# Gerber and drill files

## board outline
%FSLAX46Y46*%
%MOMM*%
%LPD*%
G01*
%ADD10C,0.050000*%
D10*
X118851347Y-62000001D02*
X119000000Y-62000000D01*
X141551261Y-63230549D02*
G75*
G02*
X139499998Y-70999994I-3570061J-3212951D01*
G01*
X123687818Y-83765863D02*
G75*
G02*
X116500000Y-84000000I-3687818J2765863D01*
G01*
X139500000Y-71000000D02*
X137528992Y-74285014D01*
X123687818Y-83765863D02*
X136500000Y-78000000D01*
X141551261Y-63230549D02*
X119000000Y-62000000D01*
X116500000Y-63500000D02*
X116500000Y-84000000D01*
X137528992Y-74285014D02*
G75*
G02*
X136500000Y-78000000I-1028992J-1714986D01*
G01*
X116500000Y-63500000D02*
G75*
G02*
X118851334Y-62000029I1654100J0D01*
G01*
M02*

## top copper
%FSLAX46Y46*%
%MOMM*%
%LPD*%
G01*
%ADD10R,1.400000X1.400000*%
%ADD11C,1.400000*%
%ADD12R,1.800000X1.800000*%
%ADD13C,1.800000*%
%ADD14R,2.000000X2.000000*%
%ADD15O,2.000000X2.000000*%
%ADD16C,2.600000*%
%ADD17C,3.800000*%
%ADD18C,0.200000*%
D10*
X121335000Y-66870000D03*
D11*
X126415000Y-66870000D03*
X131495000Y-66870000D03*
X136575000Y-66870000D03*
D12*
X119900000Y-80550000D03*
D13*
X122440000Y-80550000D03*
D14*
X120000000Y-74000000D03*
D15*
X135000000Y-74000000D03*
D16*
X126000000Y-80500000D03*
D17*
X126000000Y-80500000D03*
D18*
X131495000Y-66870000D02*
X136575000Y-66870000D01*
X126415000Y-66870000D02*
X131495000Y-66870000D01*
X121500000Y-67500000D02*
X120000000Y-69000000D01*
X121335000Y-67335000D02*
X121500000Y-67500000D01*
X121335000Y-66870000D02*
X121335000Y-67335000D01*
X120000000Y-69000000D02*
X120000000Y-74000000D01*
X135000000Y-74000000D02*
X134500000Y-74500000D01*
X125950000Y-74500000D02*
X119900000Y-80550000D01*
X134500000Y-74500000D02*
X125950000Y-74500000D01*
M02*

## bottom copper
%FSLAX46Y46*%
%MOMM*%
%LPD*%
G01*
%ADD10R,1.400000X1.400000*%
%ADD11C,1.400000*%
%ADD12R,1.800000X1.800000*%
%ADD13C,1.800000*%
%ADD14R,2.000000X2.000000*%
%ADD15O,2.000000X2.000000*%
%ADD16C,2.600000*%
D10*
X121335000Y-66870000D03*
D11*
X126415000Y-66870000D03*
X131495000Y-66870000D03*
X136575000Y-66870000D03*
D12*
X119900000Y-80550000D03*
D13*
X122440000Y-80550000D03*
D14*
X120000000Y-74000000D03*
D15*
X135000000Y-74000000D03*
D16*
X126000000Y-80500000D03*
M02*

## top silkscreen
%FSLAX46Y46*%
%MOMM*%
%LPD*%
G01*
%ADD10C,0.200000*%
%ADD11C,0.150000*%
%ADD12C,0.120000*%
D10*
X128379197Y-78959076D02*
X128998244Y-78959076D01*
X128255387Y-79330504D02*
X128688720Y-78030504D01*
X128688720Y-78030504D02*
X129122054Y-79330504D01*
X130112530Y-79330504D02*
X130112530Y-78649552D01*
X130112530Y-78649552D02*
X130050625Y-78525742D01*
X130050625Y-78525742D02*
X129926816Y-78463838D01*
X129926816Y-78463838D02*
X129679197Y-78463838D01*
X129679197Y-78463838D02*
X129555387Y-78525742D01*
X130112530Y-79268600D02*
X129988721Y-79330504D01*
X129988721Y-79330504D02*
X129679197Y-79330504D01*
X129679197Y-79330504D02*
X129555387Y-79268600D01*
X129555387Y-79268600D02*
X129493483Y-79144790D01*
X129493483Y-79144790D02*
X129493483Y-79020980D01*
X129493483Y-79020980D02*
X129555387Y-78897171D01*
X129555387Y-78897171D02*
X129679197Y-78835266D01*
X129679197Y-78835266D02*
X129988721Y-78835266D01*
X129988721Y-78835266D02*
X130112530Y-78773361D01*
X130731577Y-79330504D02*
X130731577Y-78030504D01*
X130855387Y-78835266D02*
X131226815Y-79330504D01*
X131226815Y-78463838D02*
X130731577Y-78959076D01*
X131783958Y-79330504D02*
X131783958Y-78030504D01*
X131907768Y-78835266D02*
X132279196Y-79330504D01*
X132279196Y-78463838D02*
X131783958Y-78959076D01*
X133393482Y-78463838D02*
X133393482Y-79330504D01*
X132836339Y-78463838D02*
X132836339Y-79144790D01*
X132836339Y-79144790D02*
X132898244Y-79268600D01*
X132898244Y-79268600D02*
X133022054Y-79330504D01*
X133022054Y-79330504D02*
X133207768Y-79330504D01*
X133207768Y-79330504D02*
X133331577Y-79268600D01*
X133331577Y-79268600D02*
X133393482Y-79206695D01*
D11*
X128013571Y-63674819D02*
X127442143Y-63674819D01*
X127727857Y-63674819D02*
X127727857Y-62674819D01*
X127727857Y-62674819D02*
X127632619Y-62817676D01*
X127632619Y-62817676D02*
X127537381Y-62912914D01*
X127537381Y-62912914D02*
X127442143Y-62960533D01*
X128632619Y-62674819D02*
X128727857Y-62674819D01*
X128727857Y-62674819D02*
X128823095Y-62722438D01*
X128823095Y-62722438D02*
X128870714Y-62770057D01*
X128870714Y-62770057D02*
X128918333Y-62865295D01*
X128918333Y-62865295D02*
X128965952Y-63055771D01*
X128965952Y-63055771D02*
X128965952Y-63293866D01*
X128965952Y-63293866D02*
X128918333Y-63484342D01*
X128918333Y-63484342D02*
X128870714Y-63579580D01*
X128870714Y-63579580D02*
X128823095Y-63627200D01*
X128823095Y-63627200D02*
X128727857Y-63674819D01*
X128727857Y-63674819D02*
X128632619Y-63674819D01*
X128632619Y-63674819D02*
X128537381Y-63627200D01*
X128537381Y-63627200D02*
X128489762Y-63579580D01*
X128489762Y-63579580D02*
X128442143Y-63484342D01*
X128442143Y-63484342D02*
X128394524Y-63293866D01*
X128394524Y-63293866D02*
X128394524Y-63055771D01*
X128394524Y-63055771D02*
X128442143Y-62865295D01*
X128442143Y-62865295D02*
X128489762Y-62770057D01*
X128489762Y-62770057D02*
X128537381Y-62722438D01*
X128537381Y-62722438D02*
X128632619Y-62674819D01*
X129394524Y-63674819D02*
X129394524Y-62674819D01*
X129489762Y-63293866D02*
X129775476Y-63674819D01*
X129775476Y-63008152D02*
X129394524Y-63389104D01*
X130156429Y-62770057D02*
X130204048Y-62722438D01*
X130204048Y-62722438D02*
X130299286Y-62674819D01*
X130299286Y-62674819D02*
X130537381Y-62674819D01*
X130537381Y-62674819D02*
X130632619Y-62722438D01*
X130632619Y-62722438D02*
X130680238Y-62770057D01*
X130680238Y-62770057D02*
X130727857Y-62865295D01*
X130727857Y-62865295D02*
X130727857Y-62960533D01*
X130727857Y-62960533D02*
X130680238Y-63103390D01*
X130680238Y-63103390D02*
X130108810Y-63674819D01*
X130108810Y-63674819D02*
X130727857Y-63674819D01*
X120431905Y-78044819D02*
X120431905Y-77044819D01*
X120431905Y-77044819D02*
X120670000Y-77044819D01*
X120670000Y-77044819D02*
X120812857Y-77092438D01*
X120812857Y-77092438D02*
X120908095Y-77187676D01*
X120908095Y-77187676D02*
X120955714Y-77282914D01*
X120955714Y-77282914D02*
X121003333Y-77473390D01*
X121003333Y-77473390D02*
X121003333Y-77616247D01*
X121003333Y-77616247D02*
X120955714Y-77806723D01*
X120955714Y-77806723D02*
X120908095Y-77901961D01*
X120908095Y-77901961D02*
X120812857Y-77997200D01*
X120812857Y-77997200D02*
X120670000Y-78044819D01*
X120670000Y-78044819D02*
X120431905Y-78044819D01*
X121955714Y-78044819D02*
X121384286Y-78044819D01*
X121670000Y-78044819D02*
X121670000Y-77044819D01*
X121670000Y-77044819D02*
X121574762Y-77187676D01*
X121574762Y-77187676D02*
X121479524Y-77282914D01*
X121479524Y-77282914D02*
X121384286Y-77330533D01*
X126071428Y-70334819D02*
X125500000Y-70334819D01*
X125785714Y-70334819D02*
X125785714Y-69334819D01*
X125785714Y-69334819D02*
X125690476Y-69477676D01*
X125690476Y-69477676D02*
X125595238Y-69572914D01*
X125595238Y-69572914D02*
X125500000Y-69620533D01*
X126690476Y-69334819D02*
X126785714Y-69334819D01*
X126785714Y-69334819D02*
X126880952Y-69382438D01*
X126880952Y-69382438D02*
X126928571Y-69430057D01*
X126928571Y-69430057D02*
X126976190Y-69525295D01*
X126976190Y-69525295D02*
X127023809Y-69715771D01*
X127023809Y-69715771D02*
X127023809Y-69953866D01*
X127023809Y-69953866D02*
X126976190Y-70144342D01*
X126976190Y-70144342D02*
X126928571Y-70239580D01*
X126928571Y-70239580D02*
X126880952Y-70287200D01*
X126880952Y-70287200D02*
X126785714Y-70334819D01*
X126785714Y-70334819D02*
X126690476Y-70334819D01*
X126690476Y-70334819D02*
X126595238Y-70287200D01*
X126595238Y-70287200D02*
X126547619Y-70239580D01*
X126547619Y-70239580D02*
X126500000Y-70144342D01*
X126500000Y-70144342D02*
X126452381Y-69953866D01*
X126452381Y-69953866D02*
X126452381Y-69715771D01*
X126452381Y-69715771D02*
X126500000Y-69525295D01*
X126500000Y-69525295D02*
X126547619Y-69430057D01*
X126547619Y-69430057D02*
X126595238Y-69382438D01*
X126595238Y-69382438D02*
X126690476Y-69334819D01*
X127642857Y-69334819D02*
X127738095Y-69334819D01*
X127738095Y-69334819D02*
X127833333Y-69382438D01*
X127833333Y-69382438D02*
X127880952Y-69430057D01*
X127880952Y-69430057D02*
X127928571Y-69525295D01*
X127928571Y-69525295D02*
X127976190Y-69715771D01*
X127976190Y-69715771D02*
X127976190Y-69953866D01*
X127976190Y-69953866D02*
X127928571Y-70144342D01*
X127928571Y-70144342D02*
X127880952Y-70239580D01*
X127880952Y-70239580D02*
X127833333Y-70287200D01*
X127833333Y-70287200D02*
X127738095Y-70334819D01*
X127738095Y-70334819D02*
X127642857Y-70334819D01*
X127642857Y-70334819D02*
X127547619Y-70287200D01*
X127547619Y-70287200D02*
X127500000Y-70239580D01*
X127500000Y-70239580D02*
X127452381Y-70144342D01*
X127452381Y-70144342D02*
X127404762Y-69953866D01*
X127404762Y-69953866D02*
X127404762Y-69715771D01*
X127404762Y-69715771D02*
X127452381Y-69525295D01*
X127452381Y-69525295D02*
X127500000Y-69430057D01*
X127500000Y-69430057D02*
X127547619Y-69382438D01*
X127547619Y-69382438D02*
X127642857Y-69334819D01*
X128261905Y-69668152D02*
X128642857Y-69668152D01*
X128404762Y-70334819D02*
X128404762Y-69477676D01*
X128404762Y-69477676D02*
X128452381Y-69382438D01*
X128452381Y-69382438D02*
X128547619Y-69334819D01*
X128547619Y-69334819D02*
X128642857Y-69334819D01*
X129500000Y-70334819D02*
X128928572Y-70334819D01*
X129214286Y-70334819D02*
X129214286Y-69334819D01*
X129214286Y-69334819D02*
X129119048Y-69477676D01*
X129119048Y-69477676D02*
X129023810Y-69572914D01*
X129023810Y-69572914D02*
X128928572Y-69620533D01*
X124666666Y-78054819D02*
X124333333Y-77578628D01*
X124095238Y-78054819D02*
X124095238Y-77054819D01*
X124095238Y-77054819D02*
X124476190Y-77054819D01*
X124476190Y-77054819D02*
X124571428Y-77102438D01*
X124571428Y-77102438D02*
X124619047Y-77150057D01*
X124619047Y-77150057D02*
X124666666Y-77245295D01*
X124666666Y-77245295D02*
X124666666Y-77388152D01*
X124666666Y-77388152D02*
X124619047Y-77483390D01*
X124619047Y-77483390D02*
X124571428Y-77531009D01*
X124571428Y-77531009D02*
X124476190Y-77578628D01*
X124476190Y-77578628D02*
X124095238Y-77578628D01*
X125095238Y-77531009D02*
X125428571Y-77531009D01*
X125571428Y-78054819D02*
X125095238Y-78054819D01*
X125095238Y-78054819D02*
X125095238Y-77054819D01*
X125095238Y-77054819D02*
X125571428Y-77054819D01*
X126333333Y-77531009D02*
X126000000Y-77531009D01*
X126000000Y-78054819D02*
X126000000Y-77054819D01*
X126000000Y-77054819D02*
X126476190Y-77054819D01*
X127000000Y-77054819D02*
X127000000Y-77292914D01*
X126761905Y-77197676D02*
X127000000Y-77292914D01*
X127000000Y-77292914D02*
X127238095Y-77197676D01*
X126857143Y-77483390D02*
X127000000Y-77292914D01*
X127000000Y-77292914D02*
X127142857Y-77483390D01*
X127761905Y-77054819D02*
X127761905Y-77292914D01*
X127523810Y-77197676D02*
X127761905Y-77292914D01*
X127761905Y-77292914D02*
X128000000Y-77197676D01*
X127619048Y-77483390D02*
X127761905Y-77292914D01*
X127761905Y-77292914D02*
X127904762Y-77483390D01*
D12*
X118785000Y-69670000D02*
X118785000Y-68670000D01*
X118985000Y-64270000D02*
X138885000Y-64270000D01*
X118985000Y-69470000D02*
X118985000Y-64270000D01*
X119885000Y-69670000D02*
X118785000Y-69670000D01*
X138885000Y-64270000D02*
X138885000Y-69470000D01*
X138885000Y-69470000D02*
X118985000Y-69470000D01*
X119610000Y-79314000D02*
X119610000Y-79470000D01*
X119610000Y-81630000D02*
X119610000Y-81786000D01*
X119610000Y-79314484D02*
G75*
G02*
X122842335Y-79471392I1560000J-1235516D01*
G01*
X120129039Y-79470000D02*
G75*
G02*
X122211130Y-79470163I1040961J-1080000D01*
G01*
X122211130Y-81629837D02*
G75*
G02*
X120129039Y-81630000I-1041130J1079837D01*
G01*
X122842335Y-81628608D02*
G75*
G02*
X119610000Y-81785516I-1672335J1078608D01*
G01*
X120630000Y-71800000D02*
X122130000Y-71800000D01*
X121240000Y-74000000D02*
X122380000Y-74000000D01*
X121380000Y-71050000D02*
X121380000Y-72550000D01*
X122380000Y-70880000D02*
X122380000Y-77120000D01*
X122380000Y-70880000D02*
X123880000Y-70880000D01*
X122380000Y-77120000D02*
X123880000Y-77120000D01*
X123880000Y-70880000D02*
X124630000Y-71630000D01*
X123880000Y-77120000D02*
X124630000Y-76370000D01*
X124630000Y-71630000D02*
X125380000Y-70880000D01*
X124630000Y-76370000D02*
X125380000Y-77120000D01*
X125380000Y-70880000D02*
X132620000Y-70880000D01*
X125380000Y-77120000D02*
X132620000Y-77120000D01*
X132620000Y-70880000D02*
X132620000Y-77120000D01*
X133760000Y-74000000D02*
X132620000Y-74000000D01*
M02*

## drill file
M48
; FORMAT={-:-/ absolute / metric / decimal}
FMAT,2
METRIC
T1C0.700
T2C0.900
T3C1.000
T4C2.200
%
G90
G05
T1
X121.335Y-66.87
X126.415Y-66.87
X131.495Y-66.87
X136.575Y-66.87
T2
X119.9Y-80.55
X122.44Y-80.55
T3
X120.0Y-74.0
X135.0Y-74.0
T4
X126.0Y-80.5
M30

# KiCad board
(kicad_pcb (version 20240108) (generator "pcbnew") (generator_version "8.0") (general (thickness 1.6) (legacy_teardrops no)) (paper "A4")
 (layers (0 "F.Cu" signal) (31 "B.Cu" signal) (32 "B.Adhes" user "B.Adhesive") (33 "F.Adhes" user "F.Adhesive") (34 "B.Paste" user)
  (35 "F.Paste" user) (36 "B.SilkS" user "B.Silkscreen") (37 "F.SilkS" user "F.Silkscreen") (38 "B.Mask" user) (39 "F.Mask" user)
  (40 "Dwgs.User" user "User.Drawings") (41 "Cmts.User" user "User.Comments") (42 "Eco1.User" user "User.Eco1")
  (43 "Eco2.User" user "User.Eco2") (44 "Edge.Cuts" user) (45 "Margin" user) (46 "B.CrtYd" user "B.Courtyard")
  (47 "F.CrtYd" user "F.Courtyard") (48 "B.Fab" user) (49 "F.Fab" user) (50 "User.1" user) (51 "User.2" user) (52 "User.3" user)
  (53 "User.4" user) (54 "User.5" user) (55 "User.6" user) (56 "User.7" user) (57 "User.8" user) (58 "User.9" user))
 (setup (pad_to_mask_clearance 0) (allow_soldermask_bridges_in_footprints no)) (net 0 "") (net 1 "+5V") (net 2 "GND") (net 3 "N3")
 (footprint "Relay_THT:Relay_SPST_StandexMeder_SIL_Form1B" (layer "F.Cu") (at 121.335 66.87)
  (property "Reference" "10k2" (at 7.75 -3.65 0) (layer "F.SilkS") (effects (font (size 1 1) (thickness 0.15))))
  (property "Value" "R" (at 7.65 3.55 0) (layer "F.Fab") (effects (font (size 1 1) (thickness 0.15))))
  (fp_line (start -2.55 2.8) (end -2.55 1.8) (stroke (width 0.12) (type solid)) (layer "F.SilkS"))
  (fp_line (start -2.35 -2.6) (end 17.55 -2.6) (stroke (width 0.12) (type solid)) (layer "F.SilkS"))
  (fp_line (start -2.35 2.6) (end -2.35 -2.6) (stroke (width 0.12) (type solid)) (layer "F.SilkS"))
  (fp_line (start -1.45 2.8) (end -2.55 2.8) (stroke (width 0.12) (type solid)) (layer "F.SilkS"))
  (fp_line (start 17.55 -2.6) (end 17.55 2.6) (stroke (width 0.12) (type solid)) (layer "F.SilkS"))
  (fp_line (start 17.55 2.6) (end -2.35 2.6) (stroke (width 0.12) (type solid)) (layer "F.SilkS"))
  (pad "1" thru_hole rect (at 0 0) (size 1.4 1.4) (drill 0.7) (layers "*.Cu" "*.Mask") (remove_unused_layers no) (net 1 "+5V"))
  (pad "3" thru_hole circle (at 5.08 0) (size 1.4 1.4) (drill 0.7) (layers "*.Cu" "*.Mask") (remove_unused_layers no))
  (pad "5" thru_hole circle (at 10.16 0) (size 1.4 1.4) (drill 0.7) (layers "*.Cu" "*.Mask") (remove_unused_layers no))
  (pad "7" thru_hole circle (at 15.24 0) (size 1.4 1.4) (drill 0.7) (layers "*.Cu" "*.Mask") (remove_unused_layers no)))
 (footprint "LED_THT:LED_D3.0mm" (layer "F.Cu") (at 119.9 80.55)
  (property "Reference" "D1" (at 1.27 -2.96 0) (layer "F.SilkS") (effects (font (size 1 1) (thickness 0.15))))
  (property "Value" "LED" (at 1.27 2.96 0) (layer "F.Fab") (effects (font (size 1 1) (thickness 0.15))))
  (fp_line (start -0.29 -1.236) (end -0.29 -1.08) (stroke (width 0.12) (type solid)) (layer "F.SilkS"))
  (fp_line (start -0.29 1.08) (end -0.29 1.236) (stroke (width 0.12) (type solid)) (layer "F.SilkS"))
  (fp_arc (start -0.29 -1.235516) (mid 1.366487 -1.987659) (end 2.942335 -1.078608) (stroke (width 0.12) (type solid)) (layer "F.SilkS"))
  (fp_arc (start 0.229039 -1.08) (mid 1.270117 -1.5) (end 2.31113 -1.079837) (stroke (width 0.12) (type solid)) (layer "F.SilkS"))
  (fp_arc (start 2.31113 1.079837) (mid 1.270117 1.5) (end 0.229039 1.08) (stroke (width 0.12) (type solid)) (layer "F.SilkS"))
  (fp_arc (start 2.942335 1.078608) (mid 1.366487 1.987659) (end -0.29 1.235516) (stroke (width 0.12) (type solid)) (layer "F.SilkS"))
  (pad "1" thru_hole rect (at 0 0) (size 1.8 1.8) (drill 0.9) (layers "*.Cu" "*.Mask") (remove_unused_layers no) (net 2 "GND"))
  (pad "2" thru_hole circle (at 2.54 0) (size 1.8 1.8) (drill 0.9) (layers "*.Cu" "*.Mask") (remove_unused_layers no) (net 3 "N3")))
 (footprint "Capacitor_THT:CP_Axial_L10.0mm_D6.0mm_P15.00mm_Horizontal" (layer "F.Cu") (at 120 74)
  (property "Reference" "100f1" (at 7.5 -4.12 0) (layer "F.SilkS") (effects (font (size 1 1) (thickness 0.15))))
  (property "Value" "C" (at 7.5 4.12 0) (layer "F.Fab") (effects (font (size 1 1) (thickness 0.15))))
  (fp_line (start 0.63 -2.2) (end 2.13 -2.2) (stroke (width 0.12) (type solid)) (layer "F.SilkS"))
  (fp_line (start 1.24 0) (end 2.38 0) (stroke (width 0.12) (type solid)) (layer "F.SilkS"))
  (fp_line (start 1.38 -2.95) (end 1.38 -1.45) (stroke (width 0.12) (type solid)) (layer "F.SilkS"))
  (fp_line (start 2.38 -3.12) (end 2.38 3.12) (stroke (width 0.12) (type solid)) (layer "F.SilkS"))
  (fp_line (start 2.38 -3.12) (end 3.88 -3.12) (stroke (width 0.12) (type solid)) (layer "F.SilkS"))
  (fp_line (start 2.38 3.12) (end 3.88 3.12) (stroke (width 0.12) (type solid)) (layer "F.SilkS"))
  (fp_line (start 3.88 -3.12) (end 4.63 -2.37) (stroke (width 0.12) (type solid)) (layer "F.SilkS"))
  (fp_line (start 3.88 3.12) (end 4.63 2.37) (stroke (width 0.12) (type solid)) (layer "F.SilkS"))
  (fp_line (start 4.63 -2.37) (end 5.38 -3.12) (stroke (width 0.12) (type solid)) (layer "F.SilkS"))
  (fp_line (start 4.63 2.37) (end 5.38 3.12) (stroke (width 0.12) (type solid)) (layer "F.SilkS"))
  (fp_line (start 5.38 -3.12) (end 12.62 -3.12) (stroke (width 0.12) (type solid)) (layer "F.SilkS"))
  (fp_line (start 5.38 3.12) (end 12.62 3.12) (stroke (width 0.12) (type solid)) (layer "F.SilkS"))
  (fp_line (start 12.62 -3.12) (end 12.62 3.12) (stroke (width 0.12) (type solid)) (layer "F.SilkS"))
  (fp_line (start 13.76 0) (end 12.62 0) (stroke (width 0.12) (type solid)) (layer "F.SilkS"))
  (pad "1" thru_hole rect (at 0 0) (size 2 2) (drill 1) (layers "*.Cu" "*.Mask") (remove_unused_layers no) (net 1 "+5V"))
  (pad "2" thru_hole oval (at 15 0) (size 2 2) (drill 1) (layers "*.Cu" "*.Mask") (remove_unused_layers no) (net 2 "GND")))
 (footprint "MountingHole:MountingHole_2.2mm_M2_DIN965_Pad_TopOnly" (layer "F.Cu") (at 126 80.5)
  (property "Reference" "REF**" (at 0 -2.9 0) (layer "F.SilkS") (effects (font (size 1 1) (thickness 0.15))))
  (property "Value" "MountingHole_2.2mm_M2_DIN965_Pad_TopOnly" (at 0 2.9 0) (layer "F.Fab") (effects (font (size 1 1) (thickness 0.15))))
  (pad "1" thru_hole circle (at 0 0) (size 2.6 2.6) (drill 2.2) (layers "*.Cu" "*.Mask") (remove_unused_layers no))
  (pad "1" connect circle (at 0 0) (size 3.8 3.8) (layers "F.Cu" "F.Mask")))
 (gr_line (start 118.851347 62.000001) (end 119 62) (stroke (width 0.05) (type default)) (layer "Edge.Cuts"))
 (gr_arc (start 141.551261 63.230549) (mid 142.625019 67.669547) (end 139.5 71) (stroke (width 0.05) (type default)) (layer "Edge.Cuts"))
 (gr_arc (start 123.687818 83.765863) (mid 120.15008 85.607328) (end 116.5 84) (stroke (width 0.05) (type default)) (layer "Edge.Cuts"))
 (gr_line (start 139.5 71) (end 137.528992 74.285014) (stroke (width 0.05) (type default)) (layer "Edge.Cuts"))
 (gr_line (start 123.687818 83.765863) (end 136.5 78) (stroke (width 0.05) (type default)) (layer "Edge.Cuts"))
 (gr_line (start 141.551261 63.230549) (end 119 62) (stroke (width 0.05) (type default)) (layer "Edge.Cuts"))
 (gr_line (start 116.5 63.5) (end 116.5 84) (stroke (width 0.05) (type default)) (layer "Edge.Cuts"))
 (gr_arc (start 137.528992 74.285014) (mid 138.42743 76.533867) (end 136.5 78) (stroke (width 0.05) (type default)) (layer "Edge.Cuts"))
 (gr_arc (start 116.5 63.5) (mid 117.264508 62.105472) (end 118.851347 62.000001) (stroke (width 0.05) (type default)) (layer "Edge.Cuts"))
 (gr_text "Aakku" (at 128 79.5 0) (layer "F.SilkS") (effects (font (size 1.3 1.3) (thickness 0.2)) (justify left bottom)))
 (segment (start 131.495 66.87) (end 136.575 66.87) (width 0.2) (layer "F.Cu") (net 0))
 (segment (start 126.415 66.87) (end 131.495 66.87) (width 0.2) (layer "F.Cu") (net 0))
 (segment (start 121.5 67.5) (end 120 69) (width 0.2) (layer "F.Cu") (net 1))
 (segment (start 121.335 67.335) (end 121.5 67.5) (width 0.2) (layer "F.Cu") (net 1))
 (segment (start 121.335 66.87) (end 121.335 67.335) (width 0.2) (layer "F.Cu") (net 1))
 (segment (start 120 69) (end 120 74) (width 0.2) (layer "F.Cu") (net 1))
 (segment (start 135 74) (end 134.5 74.5) (width 0.2) (layer "F.Cu") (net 2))
 (segment (start 125.95 74.5) (end 119.9 80.55) (width 0.2) (layer "F.Cu") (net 2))
 (segment (start 134.5 74.5) (end 125.95 74.5) (width 0.2) (layer "F.Cu") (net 2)))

